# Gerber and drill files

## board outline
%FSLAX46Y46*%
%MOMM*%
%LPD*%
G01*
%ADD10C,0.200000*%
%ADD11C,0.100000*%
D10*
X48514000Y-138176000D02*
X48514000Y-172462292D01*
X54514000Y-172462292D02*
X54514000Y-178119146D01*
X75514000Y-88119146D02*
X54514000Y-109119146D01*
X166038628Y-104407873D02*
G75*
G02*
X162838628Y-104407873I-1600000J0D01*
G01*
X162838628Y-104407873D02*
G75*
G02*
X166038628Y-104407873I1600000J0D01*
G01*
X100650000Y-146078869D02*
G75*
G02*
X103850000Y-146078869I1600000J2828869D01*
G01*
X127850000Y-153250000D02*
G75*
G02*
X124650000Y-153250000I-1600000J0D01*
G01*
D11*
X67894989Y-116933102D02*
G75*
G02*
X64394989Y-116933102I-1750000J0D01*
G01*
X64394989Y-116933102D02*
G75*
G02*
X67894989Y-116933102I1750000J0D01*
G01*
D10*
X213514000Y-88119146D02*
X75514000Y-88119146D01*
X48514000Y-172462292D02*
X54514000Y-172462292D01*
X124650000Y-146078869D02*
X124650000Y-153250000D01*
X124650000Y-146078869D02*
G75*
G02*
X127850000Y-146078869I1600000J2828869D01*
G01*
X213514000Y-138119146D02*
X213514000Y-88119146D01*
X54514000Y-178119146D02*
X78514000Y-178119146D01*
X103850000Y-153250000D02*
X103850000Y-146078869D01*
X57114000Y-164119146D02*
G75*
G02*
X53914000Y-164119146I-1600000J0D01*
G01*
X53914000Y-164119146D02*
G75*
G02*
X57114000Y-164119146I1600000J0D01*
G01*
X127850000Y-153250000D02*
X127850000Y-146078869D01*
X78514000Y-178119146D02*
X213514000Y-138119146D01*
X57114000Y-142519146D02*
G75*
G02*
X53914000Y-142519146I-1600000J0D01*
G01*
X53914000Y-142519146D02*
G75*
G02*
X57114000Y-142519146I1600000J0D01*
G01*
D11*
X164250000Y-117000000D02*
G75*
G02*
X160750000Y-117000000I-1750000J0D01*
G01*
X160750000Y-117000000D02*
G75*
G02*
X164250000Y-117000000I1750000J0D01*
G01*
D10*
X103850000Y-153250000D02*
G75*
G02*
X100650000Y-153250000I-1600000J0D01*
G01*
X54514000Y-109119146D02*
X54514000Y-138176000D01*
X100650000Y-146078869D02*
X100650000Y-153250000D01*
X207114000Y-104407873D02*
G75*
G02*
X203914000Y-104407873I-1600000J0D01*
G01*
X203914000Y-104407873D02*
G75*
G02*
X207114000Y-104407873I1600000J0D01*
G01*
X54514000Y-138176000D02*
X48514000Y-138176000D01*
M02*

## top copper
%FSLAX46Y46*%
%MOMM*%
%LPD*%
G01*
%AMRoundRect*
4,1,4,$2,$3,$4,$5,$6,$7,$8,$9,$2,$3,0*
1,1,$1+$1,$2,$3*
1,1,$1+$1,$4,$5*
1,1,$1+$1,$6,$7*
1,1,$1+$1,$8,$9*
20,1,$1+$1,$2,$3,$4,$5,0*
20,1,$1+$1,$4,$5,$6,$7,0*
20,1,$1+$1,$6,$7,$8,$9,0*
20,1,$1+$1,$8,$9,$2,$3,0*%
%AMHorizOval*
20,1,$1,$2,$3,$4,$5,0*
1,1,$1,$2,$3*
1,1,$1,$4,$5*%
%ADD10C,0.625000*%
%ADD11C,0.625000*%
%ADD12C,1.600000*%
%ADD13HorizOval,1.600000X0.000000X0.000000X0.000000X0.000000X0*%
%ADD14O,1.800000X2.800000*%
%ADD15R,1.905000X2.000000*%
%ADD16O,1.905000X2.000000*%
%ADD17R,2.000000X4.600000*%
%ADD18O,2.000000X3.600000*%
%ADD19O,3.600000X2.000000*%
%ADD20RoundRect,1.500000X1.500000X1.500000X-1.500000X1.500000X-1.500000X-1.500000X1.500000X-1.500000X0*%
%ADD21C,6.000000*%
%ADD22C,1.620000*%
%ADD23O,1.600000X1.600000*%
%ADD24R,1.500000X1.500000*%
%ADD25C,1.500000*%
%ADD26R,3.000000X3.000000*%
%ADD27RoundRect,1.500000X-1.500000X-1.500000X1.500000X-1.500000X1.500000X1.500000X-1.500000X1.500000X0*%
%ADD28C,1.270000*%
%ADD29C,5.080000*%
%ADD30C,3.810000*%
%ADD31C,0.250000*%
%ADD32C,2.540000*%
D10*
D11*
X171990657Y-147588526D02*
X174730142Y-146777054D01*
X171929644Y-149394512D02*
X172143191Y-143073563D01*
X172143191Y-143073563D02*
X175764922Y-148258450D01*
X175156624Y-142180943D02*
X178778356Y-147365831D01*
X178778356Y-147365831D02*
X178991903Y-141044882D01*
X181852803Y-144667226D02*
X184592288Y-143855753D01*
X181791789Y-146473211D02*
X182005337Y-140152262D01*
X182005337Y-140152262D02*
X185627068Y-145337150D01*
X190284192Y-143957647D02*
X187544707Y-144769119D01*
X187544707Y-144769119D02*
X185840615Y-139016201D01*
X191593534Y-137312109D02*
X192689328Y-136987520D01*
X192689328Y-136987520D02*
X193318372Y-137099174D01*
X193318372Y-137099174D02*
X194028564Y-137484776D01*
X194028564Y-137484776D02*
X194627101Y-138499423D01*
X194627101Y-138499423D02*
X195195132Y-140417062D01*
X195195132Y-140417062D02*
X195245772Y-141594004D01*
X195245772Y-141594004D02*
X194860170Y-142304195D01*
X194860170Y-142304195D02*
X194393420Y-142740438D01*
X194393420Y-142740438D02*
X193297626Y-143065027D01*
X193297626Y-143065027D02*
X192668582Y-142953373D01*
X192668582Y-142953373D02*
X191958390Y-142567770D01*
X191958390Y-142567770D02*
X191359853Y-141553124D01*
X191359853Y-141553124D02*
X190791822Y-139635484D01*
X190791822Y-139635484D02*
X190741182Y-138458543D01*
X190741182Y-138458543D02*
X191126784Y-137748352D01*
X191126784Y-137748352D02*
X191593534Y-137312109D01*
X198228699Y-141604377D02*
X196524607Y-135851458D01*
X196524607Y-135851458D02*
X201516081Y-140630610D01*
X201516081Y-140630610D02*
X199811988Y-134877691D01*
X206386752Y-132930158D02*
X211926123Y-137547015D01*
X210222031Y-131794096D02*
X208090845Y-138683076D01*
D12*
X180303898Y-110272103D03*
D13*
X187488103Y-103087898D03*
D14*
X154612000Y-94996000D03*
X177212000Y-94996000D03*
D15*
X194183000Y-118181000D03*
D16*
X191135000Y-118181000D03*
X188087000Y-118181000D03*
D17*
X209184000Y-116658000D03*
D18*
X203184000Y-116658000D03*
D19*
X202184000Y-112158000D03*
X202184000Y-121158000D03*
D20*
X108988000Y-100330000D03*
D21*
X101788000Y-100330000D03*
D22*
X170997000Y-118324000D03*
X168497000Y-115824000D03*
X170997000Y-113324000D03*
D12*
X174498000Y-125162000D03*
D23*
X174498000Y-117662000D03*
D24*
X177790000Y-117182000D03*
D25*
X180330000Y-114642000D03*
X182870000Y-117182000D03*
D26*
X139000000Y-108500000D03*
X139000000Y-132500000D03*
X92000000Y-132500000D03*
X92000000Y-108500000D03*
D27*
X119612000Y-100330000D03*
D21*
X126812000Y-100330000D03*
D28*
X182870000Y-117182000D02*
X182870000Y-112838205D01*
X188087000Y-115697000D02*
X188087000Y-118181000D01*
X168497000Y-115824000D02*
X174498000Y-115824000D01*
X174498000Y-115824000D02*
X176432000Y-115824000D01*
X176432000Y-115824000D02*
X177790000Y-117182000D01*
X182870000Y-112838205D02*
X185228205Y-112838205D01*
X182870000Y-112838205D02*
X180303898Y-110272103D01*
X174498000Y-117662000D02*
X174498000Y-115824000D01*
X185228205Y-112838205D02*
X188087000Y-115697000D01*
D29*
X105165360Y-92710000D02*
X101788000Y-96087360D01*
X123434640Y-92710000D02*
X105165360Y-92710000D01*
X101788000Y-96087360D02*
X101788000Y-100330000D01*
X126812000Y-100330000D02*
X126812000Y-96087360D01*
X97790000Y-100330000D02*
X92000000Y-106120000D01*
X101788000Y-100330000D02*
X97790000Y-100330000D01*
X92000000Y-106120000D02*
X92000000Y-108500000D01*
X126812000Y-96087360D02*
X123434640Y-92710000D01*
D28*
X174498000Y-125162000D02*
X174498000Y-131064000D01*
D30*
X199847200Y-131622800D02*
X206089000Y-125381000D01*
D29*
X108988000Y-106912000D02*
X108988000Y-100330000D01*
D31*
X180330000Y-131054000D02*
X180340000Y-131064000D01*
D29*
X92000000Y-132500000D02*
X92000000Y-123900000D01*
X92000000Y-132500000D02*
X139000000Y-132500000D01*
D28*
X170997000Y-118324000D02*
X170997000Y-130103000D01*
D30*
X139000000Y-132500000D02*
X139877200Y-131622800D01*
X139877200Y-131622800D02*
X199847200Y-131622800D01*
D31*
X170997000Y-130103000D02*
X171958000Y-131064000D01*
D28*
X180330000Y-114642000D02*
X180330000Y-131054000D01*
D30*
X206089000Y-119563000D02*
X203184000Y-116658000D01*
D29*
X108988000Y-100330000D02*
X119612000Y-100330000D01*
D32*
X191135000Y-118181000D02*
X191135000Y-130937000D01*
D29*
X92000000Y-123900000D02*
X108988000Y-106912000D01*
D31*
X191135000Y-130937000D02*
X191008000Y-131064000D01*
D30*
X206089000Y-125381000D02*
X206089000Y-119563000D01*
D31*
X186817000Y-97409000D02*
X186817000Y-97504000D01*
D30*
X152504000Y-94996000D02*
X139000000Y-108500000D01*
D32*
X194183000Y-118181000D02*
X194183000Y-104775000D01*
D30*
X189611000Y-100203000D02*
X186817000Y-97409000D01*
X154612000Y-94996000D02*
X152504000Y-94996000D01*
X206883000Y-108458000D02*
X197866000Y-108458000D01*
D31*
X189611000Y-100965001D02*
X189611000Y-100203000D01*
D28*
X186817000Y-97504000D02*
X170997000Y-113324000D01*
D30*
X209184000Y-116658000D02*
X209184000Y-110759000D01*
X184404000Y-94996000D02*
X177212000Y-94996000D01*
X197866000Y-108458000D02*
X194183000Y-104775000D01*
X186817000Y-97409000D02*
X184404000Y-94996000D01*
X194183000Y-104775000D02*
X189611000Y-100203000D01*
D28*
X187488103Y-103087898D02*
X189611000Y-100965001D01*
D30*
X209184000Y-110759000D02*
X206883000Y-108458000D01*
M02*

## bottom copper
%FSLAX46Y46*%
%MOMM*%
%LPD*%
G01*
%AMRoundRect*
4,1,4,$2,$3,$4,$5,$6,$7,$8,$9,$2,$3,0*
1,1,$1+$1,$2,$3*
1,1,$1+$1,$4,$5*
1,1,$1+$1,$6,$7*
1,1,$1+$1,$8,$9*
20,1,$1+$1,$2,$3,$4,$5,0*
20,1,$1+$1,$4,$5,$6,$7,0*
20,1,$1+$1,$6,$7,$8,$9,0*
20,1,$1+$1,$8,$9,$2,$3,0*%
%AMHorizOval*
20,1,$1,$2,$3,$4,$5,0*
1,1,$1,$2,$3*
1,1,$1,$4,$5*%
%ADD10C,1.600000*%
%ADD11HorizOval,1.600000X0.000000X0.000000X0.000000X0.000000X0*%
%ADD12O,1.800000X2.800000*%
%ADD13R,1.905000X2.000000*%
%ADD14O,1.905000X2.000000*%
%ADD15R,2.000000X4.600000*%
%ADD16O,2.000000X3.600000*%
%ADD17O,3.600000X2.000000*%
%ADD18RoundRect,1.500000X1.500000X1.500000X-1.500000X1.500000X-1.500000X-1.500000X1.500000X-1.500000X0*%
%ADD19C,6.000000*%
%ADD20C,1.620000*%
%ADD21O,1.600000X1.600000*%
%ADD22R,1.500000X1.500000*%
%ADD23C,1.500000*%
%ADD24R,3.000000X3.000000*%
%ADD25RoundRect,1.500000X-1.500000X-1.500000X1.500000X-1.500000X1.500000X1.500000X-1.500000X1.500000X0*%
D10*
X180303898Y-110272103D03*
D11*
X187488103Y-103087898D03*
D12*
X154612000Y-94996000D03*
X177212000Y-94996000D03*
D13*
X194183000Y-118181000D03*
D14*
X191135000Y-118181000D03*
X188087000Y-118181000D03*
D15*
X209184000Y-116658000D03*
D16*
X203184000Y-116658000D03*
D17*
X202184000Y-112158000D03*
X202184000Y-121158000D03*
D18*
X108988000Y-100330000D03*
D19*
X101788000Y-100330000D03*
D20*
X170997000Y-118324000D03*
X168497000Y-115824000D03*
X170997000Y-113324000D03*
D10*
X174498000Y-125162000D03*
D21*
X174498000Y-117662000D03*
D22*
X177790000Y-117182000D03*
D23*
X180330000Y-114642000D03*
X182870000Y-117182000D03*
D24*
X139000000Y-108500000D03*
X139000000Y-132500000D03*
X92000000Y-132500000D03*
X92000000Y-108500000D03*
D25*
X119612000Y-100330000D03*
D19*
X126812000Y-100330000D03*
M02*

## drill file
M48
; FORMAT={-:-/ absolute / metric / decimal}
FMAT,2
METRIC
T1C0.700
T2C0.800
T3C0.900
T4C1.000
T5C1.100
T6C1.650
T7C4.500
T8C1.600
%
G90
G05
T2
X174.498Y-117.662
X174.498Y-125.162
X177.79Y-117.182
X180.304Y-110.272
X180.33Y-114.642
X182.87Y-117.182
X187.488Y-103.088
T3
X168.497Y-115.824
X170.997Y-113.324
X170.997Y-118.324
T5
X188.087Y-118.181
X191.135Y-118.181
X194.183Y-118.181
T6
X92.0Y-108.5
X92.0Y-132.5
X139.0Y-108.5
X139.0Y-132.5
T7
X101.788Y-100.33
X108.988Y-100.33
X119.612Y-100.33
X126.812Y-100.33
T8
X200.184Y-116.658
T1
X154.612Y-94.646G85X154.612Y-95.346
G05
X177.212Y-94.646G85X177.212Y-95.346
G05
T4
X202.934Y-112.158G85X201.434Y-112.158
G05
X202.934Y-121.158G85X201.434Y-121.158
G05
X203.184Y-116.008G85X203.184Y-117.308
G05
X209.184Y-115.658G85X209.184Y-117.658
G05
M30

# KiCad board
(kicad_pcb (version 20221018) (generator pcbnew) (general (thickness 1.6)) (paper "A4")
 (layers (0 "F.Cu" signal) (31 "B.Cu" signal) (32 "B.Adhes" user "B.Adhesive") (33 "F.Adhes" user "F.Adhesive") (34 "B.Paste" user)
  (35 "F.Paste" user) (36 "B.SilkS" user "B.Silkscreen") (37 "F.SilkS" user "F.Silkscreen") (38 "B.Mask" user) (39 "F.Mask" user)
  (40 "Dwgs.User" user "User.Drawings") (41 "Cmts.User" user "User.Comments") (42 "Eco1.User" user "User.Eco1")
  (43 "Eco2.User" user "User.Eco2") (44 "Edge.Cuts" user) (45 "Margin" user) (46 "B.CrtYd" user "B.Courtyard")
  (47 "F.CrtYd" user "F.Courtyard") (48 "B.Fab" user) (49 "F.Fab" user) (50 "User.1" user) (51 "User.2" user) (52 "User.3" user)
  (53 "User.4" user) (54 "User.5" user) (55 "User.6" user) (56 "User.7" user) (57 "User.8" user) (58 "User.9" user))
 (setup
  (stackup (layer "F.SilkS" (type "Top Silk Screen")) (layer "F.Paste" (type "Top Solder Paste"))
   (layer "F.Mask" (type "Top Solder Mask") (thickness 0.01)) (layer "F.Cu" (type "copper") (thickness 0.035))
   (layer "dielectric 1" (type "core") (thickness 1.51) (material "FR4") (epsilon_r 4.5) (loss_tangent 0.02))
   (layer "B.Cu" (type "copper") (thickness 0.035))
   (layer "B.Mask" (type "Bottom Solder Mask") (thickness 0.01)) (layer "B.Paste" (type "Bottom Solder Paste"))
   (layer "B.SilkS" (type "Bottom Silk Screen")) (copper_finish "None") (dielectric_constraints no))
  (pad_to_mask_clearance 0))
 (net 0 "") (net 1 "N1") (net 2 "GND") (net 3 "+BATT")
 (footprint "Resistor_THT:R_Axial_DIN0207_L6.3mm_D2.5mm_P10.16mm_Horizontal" (layer "F.Cu") (at 180.303898 110.272103 45)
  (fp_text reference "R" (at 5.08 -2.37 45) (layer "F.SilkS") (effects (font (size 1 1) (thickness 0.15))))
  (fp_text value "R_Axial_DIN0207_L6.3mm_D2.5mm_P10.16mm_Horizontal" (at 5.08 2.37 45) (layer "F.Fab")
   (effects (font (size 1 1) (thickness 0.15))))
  (pad "1" thru_hole circle (at 0 0 45) (size 1.6 1.6) (drill 0.8) (layers "*.Cu" "*.Mask"))
  (pad "2" thru_hole oval (at 10.16 0 45) (size 1.6 1.6) (drill 0.8) (layers "*.Cu" "*.Mask") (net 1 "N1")))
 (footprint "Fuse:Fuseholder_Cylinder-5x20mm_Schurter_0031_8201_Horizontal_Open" (layer "F.Cu") (at 154.612 94.996)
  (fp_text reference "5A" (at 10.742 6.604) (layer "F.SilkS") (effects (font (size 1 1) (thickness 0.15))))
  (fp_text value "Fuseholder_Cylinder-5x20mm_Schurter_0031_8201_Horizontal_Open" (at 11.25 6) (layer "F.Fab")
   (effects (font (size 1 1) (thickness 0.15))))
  (pad "1" thru_hole oval (at 0 0) (size 1.8 2.8) (drill oval 0.7 1.4) (layers "*.Cu" "*.Mask") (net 1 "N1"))
  (pad "2" thru_hole oval (at 22.6 0) (size 1.8 2.8) (drill oval 0.7 1.4) (layers "*.Cu" "*.Mask") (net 1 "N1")))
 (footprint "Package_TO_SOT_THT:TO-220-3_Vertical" (layer "F.Cu") (at 194.183 118.181 180)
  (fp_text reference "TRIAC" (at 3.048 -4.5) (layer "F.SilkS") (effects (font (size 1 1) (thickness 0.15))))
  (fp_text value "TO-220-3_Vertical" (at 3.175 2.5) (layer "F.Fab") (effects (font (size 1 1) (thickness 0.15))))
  (pad "1" thru_hole rect (at 0 0 180) (size 1.905 2) (drill 1.1) (layers "*.Cu" "*.Mask") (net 1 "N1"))
  (pad "2" thru_hole oval (at 3.048 0 180) (size 1.905 2) (drill 1.1) (layers "*.Cu" "*.Mask") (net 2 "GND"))
  (pad "3" thru_hole oval (at 6.096 0 180) (size 1.905 2) (drill 1.1) (layers "*.Cu" "*.Mask")))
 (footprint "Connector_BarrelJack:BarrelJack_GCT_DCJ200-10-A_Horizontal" (layer "F.Cu") (at 209.184 116.658 -90)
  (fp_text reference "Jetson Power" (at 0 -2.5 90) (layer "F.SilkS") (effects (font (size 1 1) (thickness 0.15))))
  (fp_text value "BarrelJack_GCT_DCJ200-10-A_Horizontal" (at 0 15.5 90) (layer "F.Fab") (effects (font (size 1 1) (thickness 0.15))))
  (pad "" np_thru_hole circle (at 0 9 270) (size 1.6 1.6) (drill 1.6) (layers "F&B.Cu" "*.Mask"))
  (pad "1" thru_hole rect (at 0 0 270) (size 4.6 2) (drill oval 3 1) (layers "*.Cu" "*.Mask") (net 1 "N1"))
  (pad "2" thru_hole oval (at 0 6 270) (size 3.6 2) (drill oval 2.3 1) (layers "*.Cu" "*.Mask") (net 2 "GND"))
  (pad "MS" thru_hole oval (at -4.5 7 270) (size 2 3.6) (drill oval 1 2.5) (layers "*.Cu" "*.Mask"))
  (pad "MS" thru_hole oval (at 4.5 7 270) (size 2 3.6) (drill oval 1 2.5) (layers "*.Cu" "*.Mask")))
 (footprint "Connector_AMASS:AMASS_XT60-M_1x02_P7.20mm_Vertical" (layer "F.Cu") (at 108.988 100.33 180)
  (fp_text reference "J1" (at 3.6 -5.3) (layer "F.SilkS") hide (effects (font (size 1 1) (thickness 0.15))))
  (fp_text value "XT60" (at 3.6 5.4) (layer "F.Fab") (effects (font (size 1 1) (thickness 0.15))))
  (pad "1" thru_hole roundrect (at 0 0 180) (size 6 6) (drill 4.5) (layers "*.Cu" "*.Mask") (roundrect_rratio 0.25) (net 2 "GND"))
  (pad "2" thru_hole circle (at 7.2 0 180) (size 6 6) (drill 4.5) (layers "*.Cu" "*.Mask") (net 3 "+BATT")))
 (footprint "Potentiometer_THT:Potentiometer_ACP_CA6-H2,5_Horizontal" (layer "F.Cu") (at 170.997 118.324 180)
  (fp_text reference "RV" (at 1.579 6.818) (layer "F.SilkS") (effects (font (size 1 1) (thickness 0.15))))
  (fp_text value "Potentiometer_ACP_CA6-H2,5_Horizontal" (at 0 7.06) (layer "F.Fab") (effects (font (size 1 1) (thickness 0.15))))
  (pad "1" thru_hole circle (at 0 0 180) (size 1.62 1.62) (drill 0.9) (layers "*.Cu" "*.Mask") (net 2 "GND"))
  (pad "2" thru_hole circle (at 2.5 2.5 180) (size 1.62 1.62) (drill 0.9) (layers "*.Cu" "*.Mask"))
  (pad "3" thru_hole circle (at 0 5 180) (size 1.62 1.62) (drill 0.9) (layers "*.Cu" "*.Mask") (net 1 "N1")))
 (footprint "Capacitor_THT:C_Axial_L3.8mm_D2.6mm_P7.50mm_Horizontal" (layer "F.Cu") (at 174.498 125.162 90)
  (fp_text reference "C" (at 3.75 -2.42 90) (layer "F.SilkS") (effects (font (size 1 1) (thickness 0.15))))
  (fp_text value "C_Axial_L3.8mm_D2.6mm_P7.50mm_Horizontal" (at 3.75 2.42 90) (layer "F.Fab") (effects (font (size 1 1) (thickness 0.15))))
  (pad "1" thru_hole circle (at 0 0 90) (size 1.6 1.6) (drill 0.8) (layers "*.Cu" "*.Mask") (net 2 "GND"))
  (pad "2" thru_hole oval (at 7.5 0 90) (size 1.6 1.6) (drill 0.8) (layers "*.Cu" "*.Mask")))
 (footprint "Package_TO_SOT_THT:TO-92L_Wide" (layer "F.Cu") (at 177.79 117.182)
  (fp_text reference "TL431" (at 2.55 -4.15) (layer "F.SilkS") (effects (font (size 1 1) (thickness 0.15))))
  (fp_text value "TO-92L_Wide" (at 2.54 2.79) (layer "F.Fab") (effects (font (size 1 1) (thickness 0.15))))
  (pad "1" thru_hole rect (at 0 0) (size 1.5 1.5) (drill 0.8) (layers "*.Cu" "*.Mask"))
  (pad "2" thru_hole circle (at 2.54 -2.54) (size 1.5 1.5) (drill 0.8) (layers "*.Cu" "*.Mask") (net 2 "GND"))
  (pad "3" thru_hole circle (at 5.08 0) (size 1.5 1.5) (drill 0.8) (layers "*.Cu" "*.Mask")))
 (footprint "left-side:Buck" (layer "B.Cu") (at 115.5 120.5 180)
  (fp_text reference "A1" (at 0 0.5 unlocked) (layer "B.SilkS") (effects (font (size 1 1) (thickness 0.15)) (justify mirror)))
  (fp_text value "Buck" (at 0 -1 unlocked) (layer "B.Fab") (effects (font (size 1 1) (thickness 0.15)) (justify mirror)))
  (pad "1" thru_hole rect (at -23.5 12 180) (size 3 3) (drill 1.65) (layers "*.Cu" "*.Mask") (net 1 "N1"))
  (pad "2" thru_hole rect (at -23.5 -12 180) (size 3 3) (drill 1.65) (layers "*.Cu" "*.Mask") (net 2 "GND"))
  (pad "3" thru_hole rect (at 23.5 -12 180) (size 3 3) (drill 1.65) (layers "*.Cu" "*.Mask") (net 2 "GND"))
  (pad "4" thru_hole rect (at 23.5 12 180) (size 3 3) (drill 1.65) (layers "*.Cu" "*.Mask") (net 3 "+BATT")))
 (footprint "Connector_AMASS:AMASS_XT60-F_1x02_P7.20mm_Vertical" (layer "B.Cu") (at 119.612 100.33)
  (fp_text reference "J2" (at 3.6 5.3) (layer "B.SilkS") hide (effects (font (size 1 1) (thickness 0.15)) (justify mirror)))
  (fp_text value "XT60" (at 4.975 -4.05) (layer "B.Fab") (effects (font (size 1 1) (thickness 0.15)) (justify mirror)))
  (pad "1" thru_hole roundrect (at 0 0) (size 6 6) (drill 4.5) (layers "*.Cu" "*.Mask") (roundrect_rratio 0.25) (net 2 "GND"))
  (pad "2" thru_hole circle (at 7.2 0) (size 6 6) (drill 4.5) (layers "*.Cu" "*.Mask") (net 3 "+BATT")))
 (gr_line (start 48.514 138.176) (end 48.514 172.462292) (stroke (width 0.2) (type solid)) (layer "Edge.Cuts"))
 (gr_line (start 54.514 172.462292) (end 54.514 178.119146) (stroke (width 0.2) (type solid)) (layer "Edge.Cuts"))
 (gr_line (start 75.514 88.119146) (end 54.514 109.119146) (stroke (width 0.2) (type solid)) (layer "Edge.Cuts"))
 (gr_circle (center 164.438628 104.407873) (end 166.038628 104.407873) (stroke (width 0.2) (type solid)) (fill none) (layer "Edge.Cuts"))
 (gr_arc (start 100.65 146.078869) (mid 102.25 140) (end 103.85 146.078869) (stroke (width 0.2) (type solid)) (layer "Edge.Cuts"))
 (gr_arc (start 127.85 153.25) (mid 126.25 154.85) (end 124.65 153.25) (stroke (width 0.2) (type solid)) (layer "Edge.Cuts"))
 (gr_circle (center 66.144989 116.933102) (end 67.894989 116.933102) (stroke (width 0.1) (type default)) (fill none) (layer "Edge.Cuts"))
 (gr_line (start 213.514 88.119146) (end 75.514 88.119146) (stroke (width 0.2) (type solid)) (layer "Edge.Cuts"))
 (gr_line (start 48.514 172.462292) (end 54.514 172.462292) (stroke (width 0.2) (type solid)) (layer "Edge.Cuts"))
 (gr_line (start 124.65 146.078869) (end 124.65 153.25) (stroke (width 0.2) (type solid)) (layer "Edge.Cuts"))
 (gr_arc (start 124.65 146.078869) (mid 126.25 140) (end 127.85 146.078869) (stroke (width 0.2) (type solid)) (layer "Edge.Cuts"))
 (gr_line (start 213.514 138.119146) (end 213.514 88.119146) (stroke (width 0.2) (type solid)) (layer "Edge.Cuts"))
 (gr_line (start 54.514 178.119146) (end 78.514 178.119146) (stroke (width 0.2) (type solid)) (layer "Edge.Cuts"))
 (gr_line (start 103.85 153.25) (end 103.85 146.078869) (stroke (width 0.2) (type solid)) (layer "Edge.Cuts"))
 (gr_circle (center 55.514 164.119146) (end 57.114 164.119146) (stroke (width 0.2) (type solid)) (fill none) (layer "Edge.Cuts"))
 (gr_line (start 127.85 153.25) (end 127.85 146.078869) (stroke (width 0.2) (type solid)) (layer "Edge.Cuts"))
 (gr_line (start 78.514 178.119146) (end 213.514 138.119146) (stroke (width 0.2) (type solid)) (layer "Edge.Cuts"))
 (gr_circle (center 55.514 142.519146) (end 57.114 142.519146) (stroke (width 0.2) (type solid)) (fill none) (layer "Edge.Cuts"))
 (gr_circle (center 162.5 117) (end 164.25 117) (stroke (width 0.1) (type default)) (fill none) (layer "Edge.Cuts"))
 (gr_arc (start 103.85 153.25) (mid 102.25 154.85) (end 100.65 153.25) (stroke (width 0.2) (type solid)) (layer "Edge.Cuts"))
 (gr_line (start 54.514 109.119146) (end 54.514 138.176) (stroke (width 0.2) (type solid)) (layer "Edge.Cuts"))
 (gr_line (start 100.65 146.078869) (end 100.65 153.25) (stroke (width 0.2) (type solid)) (layer "Edge.Cuts"))
 (gr_circle (center 205.514 104.407873) (end 207.114 104.407873) (stroke (width 0.2) (type solid)) (fill none) (layer "Edge.Cuts"))
 (gr_line (start 54.514 138.176) (end 48.514 138.176) (stroke (width 0.2) (type solid)) (layer "Edge.Cuts"))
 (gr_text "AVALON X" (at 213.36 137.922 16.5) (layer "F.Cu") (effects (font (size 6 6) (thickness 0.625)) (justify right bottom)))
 (segment (start 182.87 117.182) (end 182.87 112.838205) (width 1.27) (layer "F.Cu") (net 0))
 (segment (start 188.087 115.697) (end 188.087 118.181) (width 1.27) (layer "F.Cu") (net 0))
 (segment (start 168.497 115.824) (end 174.498 115.824) (width 1.27) (layer "F.Cu") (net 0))
 (segment (start 174.498 115.824) (end 176.432 115.824) (width 1.27) (layer "F.Cu") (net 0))
 (segment (start 176.432 115.824) (end 177.79 117.182) (width 1.27) (layer "F.Cu") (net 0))
 (segment (start 182.87 112.838205) (end 185.228205 112.838205) (width 1.27) (layer "F.Cu") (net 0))
 (segment (start 182.87 112.838205) (end 180.303898 110.272103) (width 1.27) (layer "F.Cu") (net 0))
 (segment (start 174.498 117.662) (end 174.498 115.824) (width 1.27) (layer "F.Cu") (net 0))
 (segment (start 185.228205 112.838205) (end 188.087 115.697) (width 1.27) (layer "F.Cu") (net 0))
 (segment (start 105.16536 92.71) (end 101.788 96.08736) (width 5.08) (layer "F.Cu") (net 3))
 (segment (start 123.43464 92.71) (end 105.16536 92.71) (width 5.08) (layer "F.Cu") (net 3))
 (segment (start 101.788 96.08736) (end 101.788 100.33) (width 5.08) (layer "F.Cu") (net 3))
 (segment (start 126.812 100.33) (end 126.812 96.08736) (width 5.08) (layer "F.Cu") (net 3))
 (segment (start 97.79 100.33) (end 92 106.12) (width 5.08) (layer "F.Cu") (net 3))
 (segment (start 101.788 100.33) (end 97.79 100.33) (width 5.08) (layer "F.Cu") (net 3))
 (segment (start 92 106.12) (end 92 108.5) (width 5.08) (layer "F.Cu") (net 3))
 (segment (start 126.812 96.08736) (end 123.43464 92.71) (width 5.08) (layer "F.Cu") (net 3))
 (segment (start 174.498 125.162) (end 174.498 131.064) (width 1.27) (layer "F.Cu") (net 2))
 (segment (start 199.8472 131.6228) (end 206.089 125.381) (width 3.81) (layer "F.Cu") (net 2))
 (segment (start 108.988 106.912) (end 108.988 100.33) (width 5.08) (layer "F.Cu") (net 2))
 (segment (start 180.33 131.054) (end 180.34 131.064) (width 0.25) (layer "F.Cu") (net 2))
 (segment (start 92 132.5) (end 92 123.9) (width 5.08) (layer "F.Cu") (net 2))
 (segment (start 92 132.5) (end 139 132.5) (width 5.08) (layer "F.Cu") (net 2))
 (segment (start 170.997 118.324) (end 170.997 130.103) (width 1.27) (layer "F.Cu") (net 2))
 (segment (start 139 132.5) (end 139.8772 131.6228) (width 3.81) (layer "F.Cu") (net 2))
 (segment (start 139.8772 131.6228) (end 199.8472 131.6228) (width 3.81) (layer "F.Cu") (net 2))
 (segment (start 170.997 130.103) (end 171.958 131.064) (width 0.25) (layer "F.Cu") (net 2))
 (segment (start 180.33 114.642) (end 180.33 131.054) (width 1.27) (layer "F.Cu") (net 2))
 (segment (start 206.089 119.563) (end 203.184 116.658) (width 3.81) (layer "F.Cu") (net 2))
 (segment (start 108.988 100.33) (end 119.612 100.33) (width 5.08) (layer "F.Cu") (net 2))
 (segment (start 191.135 118.181) (end 191.135 130.937) (width 2.54) (layer "F.Cu") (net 2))
 (segment (start 92 123.9) (end 108.988 106.912) (width 5.08) (layer "F.Cu") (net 2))
 (segment (start 191.135 130.937) (end 191.008 131.064) (width 0.25) (layer "F.Cu") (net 2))
 (segment (start 206.089 125.381) (end 206.089 119.563) (width 3.81) (layer "F.Cu") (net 2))
 (segment (start 186.817 97.409) (end 186.817 97.504) (width 0.25) (layer "F.Cu") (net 1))
 (segment (start 152.504 94.996) (end 139 108.5) (width 3.81) (layer "F.Cu") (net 1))
 (segment (start 194.183 118.181) (end 194.183 104.775) (width 2.54) (layer "F.Cu") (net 1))
 (segment (start 189.611 100.203) (end 186.817 97.409) (width 3.81) (layer "F.Cu") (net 1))
 (segment (start 154.612 94.996) (end 152.504 94.996) (width 3.81) (layer "F.Cu") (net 1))
 (segment (start 206.883 108.458) (end 197.866 108.458) (width 3.81) (layer "F.Cu") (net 1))
 (segment (start 189.611 100.965001) (end 189.611 100.203) (width 0.25) (layer "F.Cu") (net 1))
 (segment (start 186.817 97.504) (end 170.997 113.324) (width 1.27) (layer "F.Cu") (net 1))
 (segment (start 209.184 116.658) (end 209.184 110.759) (width 3.81) (layer "F.Cu") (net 1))
 (segment (start 184.404 94.996) (end 177.212 94.996) (width 3.81) (layer "F.Cu") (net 1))
 (segment (start 197.866 108.458) (end 194.183 104.775) (width 3.81) (layer "F.Cu") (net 1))
 (segment (start 186.817 97.409) (end 184.404 94.996) (width 3.81) (layer "F.Cu") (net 1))
 (segment (start 194.183 104.775) (end 189.611 100.203) (width 3.81) (layer "F.Cu") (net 1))
 (segment (start 187.488103 103.087898) (end 189.611 100.965001) (width 1.27) (layer "F.Cu") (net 1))
 (segment (start 209.184 110.759) (end 206.883 108.458) (width 3.81) (layer "F.Cu") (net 1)))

